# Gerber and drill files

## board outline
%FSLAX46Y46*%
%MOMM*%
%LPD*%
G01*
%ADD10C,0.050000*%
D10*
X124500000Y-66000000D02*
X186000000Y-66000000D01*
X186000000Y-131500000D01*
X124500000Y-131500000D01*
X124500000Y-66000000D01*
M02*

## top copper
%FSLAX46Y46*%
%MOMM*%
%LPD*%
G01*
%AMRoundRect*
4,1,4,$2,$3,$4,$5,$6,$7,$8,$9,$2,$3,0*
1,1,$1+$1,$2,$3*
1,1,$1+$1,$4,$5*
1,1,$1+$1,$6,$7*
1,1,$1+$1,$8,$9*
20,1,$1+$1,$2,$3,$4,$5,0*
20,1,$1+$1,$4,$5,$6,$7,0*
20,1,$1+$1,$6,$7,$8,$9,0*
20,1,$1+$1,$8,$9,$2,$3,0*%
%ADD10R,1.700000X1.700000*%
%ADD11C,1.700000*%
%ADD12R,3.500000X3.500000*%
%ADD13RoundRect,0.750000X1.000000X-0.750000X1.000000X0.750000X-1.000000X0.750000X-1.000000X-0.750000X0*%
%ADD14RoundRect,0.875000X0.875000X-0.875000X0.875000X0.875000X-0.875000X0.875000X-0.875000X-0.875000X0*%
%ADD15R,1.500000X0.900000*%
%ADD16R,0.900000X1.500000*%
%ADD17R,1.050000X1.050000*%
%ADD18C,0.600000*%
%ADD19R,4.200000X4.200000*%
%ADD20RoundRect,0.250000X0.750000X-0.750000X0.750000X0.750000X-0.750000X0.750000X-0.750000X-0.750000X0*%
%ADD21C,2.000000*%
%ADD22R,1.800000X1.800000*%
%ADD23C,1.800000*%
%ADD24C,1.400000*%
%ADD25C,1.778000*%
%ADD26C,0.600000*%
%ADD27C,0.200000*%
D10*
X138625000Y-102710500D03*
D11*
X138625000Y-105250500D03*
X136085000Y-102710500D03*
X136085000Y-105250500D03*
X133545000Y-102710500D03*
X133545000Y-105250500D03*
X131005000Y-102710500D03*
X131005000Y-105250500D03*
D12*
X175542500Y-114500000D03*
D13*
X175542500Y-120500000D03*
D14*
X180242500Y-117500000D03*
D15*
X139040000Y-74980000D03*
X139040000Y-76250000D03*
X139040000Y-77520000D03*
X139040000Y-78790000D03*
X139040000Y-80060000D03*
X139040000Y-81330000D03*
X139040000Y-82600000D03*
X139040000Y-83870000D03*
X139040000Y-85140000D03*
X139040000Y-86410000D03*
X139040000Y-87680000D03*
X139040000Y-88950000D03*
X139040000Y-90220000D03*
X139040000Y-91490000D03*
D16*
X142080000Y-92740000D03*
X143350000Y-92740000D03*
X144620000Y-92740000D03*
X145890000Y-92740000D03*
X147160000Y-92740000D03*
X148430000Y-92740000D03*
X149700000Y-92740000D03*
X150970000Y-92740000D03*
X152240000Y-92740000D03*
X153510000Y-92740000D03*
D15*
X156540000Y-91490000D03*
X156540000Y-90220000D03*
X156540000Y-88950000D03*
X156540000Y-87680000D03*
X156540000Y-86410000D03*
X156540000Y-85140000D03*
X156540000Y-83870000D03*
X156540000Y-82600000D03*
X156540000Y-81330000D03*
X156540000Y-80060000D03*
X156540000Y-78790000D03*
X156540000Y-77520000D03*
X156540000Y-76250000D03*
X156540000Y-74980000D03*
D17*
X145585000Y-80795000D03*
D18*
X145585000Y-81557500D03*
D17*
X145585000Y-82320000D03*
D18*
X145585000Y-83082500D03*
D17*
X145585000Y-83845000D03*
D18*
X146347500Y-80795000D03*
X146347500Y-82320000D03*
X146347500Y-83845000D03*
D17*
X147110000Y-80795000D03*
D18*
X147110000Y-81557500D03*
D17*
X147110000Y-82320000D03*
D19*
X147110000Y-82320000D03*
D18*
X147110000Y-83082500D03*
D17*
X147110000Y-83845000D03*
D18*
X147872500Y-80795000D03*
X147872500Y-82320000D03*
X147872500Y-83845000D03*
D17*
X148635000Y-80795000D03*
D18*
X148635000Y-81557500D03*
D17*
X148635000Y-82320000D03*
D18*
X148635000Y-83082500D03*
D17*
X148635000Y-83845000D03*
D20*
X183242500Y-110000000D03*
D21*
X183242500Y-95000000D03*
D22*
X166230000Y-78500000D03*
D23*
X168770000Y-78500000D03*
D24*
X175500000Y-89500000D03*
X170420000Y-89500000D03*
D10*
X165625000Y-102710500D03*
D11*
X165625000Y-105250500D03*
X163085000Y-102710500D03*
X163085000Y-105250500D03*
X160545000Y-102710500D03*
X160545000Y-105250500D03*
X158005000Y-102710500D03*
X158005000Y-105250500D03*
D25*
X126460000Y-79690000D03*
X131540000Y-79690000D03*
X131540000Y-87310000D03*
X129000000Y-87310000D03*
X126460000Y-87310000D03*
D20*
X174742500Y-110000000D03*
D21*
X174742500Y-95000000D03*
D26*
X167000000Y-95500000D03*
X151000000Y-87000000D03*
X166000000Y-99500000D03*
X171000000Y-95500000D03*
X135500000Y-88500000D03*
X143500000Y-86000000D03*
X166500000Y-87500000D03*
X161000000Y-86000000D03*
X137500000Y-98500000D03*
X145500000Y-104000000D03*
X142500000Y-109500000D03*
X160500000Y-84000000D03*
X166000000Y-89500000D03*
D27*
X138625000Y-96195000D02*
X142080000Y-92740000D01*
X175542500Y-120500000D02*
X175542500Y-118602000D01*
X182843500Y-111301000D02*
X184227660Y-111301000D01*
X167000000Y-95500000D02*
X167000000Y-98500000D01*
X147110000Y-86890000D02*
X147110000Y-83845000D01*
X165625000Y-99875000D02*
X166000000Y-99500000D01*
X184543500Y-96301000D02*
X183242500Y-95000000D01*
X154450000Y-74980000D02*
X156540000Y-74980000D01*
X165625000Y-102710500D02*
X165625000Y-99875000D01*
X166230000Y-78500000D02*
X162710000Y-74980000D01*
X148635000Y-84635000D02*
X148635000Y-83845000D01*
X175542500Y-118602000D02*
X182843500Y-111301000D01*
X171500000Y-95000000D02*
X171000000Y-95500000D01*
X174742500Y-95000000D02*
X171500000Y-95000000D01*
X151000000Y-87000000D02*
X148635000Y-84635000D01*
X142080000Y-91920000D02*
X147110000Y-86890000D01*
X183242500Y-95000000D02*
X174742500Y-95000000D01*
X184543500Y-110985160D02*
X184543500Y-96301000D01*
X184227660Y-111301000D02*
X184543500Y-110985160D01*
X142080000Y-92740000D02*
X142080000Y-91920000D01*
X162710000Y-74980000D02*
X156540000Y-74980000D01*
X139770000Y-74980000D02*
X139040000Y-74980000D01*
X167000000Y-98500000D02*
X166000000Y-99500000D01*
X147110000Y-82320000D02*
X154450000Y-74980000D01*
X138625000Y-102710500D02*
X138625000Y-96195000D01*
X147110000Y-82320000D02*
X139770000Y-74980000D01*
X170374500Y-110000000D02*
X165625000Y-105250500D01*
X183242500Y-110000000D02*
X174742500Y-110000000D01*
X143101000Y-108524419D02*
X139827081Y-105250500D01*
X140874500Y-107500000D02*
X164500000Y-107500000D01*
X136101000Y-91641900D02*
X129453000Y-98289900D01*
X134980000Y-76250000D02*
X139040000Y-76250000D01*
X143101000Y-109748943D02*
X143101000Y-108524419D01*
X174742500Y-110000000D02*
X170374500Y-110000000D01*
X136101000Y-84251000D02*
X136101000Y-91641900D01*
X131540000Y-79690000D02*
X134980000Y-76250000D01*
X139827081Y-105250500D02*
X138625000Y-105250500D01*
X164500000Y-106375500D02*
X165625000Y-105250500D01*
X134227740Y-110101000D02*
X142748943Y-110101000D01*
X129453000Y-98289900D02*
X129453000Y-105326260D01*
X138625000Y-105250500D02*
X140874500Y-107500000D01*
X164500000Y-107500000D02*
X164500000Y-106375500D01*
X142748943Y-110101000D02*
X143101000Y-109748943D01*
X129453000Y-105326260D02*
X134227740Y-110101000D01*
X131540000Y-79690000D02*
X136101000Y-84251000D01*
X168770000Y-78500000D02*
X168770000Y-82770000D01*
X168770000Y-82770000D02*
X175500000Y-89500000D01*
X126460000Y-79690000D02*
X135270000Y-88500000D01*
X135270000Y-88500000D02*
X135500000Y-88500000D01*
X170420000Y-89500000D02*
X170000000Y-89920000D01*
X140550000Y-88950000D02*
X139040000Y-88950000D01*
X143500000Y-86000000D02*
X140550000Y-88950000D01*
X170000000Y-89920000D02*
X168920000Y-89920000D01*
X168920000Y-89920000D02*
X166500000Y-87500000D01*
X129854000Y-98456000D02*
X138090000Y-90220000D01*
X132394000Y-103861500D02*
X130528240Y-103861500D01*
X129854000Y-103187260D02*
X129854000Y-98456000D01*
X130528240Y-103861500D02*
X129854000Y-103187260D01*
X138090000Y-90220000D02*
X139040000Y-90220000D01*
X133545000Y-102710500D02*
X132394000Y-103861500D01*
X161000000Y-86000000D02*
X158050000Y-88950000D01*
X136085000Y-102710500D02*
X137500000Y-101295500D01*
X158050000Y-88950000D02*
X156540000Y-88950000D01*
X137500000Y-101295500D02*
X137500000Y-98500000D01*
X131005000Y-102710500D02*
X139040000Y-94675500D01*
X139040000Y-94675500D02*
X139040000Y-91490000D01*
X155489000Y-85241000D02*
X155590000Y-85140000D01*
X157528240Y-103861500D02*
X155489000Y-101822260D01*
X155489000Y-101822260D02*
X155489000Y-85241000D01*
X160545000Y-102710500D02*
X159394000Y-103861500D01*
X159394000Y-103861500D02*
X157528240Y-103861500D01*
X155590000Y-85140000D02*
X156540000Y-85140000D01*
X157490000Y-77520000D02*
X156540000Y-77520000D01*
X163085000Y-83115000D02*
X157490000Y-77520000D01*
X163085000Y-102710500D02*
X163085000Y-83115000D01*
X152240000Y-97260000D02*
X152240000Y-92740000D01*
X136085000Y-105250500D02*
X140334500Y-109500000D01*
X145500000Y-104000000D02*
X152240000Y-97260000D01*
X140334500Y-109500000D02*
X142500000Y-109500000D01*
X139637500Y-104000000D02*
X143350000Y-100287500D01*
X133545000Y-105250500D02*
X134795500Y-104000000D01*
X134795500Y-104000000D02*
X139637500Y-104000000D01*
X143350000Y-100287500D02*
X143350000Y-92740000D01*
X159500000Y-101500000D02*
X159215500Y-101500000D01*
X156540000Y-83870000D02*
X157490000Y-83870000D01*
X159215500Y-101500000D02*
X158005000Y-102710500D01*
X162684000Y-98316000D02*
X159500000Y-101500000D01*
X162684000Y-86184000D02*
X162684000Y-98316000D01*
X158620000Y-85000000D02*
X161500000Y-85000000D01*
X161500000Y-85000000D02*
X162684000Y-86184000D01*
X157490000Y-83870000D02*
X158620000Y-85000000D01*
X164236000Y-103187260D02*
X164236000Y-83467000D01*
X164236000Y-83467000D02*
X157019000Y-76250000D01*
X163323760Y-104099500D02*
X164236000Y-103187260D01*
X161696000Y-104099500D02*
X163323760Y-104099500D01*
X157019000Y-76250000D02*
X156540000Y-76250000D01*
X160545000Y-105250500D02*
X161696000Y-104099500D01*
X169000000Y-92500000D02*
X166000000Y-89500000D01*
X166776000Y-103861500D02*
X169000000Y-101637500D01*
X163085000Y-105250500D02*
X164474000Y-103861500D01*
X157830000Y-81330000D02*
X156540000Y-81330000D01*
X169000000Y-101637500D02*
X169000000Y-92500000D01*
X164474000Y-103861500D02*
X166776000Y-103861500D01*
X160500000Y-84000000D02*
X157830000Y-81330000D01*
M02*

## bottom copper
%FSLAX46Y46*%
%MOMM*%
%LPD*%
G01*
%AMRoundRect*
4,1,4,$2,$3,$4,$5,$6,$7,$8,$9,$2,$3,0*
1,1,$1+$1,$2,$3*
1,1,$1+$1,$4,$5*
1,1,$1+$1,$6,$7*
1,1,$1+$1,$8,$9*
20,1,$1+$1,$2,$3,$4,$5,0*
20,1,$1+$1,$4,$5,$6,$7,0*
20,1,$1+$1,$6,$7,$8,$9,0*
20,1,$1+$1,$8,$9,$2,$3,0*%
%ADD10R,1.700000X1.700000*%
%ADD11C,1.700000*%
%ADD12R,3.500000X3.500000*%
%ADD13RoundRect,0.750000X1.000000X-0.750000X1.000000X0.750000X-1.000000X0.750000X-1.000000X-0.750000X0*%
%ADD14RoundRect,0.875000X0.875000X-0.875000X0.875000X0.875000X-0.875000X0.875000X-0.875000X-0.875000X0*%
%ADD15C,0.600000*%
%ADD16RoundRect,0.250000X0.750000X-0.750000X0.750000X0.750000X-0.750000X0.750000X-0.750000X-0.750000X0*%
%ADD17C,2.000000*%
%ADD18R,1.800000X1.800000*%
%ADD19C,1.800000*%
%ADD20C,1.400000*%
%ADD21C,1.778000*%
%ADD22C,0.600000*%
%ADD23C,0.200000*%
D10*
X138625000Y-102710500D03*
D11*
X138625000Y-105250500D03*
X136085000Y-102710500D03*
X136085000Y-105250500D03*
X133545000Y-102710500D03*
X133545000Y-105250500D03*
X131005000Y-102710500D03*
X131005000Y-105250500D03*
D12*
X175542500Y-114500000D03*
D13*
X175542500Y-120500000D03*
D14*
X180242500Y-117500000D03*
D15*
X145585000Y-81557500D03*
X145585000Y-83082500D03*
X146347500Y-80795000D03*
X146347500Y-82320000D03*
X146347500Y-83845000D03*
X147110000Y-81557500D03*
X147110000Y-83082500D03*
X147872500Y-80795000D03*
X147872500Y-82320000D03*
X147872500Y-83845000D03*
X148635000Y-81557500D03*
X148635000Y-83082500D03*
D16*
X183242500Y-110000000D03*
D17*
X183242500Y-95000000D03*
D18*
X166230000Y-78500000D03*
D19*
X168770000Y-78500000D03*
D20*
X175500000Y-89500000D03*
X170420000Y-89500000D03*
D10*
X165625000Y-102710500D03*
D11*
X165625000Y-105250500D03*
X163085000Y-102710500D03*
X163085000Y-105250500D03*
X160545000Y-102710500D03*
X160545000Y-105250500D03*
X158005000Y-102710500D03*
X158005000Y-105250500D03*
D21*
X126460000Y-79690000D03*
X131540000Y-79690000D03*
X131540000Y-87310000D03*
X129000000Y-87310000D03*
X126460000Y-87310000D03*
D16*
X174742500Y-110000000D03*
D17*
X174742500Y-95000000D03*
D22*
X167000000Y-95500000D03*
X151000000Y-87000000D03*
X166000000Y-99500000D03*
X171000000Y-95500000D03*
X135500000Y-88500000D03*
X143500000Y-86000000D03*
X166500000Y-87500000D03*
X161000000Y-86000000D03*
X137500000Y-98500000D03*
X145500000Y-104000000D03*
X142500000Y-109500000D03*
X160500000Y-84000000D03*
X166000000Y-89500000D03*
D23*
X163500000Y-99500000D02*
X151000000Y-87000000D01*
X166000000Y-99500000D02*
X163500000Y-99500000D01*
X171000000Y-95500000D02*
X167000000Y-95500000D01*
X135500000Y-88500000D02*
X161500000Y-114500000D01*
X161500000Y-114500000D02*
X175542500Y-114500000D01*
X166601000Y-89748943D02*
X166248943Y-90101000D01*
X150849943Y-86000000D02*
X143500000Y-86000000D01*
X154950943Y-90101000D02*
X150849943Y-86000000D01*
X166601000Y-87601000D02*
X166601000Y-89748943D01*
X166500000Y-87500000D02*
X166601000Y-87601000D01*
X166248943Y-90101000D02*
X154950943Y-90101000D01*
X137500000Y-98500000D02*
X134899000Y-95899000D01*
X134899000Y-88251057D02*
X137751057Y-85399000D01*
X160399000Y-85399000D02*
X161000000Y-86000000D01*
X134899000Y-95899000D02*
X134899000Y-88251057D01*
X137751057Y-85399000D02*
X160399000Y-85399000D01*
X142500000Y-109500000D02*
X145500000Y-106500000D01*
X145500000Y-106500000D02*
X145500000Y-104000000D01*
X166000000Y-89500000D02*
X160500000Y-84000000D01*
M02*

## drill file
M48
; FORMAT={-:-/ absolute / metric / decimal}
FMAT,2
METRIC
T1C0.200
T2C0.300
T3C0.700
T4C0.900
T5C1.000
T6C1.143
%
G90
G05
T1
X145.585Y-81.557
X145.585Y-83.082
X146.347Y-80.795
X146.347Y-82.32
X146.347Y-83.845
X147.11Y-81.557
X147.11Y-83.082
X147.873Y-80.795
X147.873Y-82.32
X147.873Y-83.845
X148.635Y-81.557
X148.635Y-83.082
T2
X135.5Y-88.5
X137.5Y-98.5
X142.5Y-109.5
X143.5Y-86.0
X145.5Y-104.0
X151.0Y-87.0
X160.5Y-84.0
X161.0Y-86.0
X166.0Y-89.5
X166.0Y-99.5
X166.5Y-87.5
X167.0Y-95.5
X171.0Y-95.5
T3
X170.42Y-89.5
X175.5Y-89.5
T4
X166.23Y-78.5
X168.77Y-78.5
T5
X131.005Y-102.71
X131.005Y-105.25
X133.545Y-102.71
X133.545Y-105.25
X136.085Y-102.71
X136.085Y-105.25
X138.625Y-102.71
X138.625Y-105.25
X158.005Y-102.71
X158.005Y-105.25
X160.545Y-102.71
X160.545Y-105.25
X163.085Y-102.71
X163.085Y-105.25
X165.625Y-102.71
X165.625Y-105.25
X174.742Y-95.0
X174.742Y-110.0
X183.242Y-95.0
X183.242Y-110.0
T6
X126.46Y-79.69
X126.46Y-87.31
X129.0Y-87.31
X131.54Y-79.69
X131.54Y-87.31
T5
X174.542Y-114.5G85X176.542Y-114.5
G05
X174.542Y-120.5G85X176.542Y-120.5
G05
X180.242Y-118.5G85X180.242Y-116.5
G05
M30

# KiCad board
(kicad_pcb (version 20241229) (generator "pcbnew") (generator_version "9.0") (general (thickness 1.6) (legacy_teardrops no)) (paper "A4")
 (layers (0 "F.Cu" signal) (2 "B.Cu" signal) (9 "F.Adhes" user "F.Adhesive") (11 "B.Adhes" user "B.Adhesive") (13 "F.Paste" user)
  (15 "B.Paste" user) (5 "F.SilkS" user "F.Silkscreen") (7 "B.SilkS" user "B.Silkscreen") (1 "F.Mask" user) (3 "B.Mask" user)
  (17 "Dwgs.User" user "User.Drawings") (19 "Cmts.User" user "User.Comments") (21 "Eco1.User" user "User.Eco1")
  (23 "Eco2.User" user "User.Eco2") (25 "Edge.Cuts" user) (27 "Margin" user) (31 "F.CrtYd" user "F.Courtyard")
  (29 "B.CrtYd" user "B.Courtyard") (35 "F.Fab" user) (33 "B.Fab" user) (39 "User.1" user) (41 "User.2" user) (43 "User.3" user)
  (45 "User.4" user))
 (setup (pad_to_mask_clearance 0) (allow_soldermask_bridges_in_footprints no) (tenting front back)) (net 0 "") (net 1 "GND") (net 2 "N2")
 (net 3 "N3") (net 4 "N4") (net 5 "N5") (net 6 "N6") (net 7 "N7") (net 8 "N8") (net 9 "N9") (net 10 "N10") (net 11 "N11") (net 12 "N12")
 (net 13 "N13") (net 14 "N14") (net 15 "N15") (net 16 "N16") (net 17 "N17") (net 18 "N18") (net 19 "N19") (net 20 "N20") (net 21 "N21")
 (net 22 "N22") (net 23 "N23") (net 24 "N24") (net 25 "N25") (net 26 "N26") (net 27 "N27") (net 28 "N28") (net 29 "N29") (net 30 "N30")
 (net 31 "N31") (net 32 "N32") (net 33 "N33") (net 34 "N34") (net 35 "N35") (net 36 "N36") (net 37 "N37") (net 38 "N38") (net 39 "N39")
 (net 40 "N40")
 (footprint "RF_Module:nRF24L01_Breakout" (layer "F.Cu") (at 138.625 102.7105 -90)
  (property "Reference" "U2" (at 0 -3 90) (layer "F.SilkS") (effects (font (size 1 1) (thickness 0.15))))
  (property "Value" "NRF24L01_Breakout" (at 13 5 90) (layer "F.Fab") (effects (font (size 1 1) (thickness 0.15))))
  (pad "1" thru_hole rect (at 0 0 270) (size 1.7 1.7) (drill 1) (layers "*.Cu" "*.Mask") (remove_unused_layers no) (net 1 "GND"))
  (pad "2" thru_hole circle (at 2.54 0 270) (size 1.7 1.7) (drill 1) (layers "*.Cu" "*.Mask") (remove_unused_layers no) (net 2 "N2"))
  (pad "3" thru_hole circle (at 0 2.54 270) (size 1.7 1.7) (drill 1) (layers "*.Cu" "*.Mask") (remove_unused_layers no) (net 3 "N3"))
  (pad "4" thru_hole circle (at 2.54 2.54 270) (size 1.7 1.7) (drill 1) (layers "*.Cu" "*.Mask") (remove_unused_layers no) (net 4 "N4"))
  (pad "5" thru_hole circle (at 0 5.08 270) (size 1.7 1.7) (drill 1) (layers "*.Cu" "*.Mask") (remove_unused_layers no) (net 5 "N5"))
  (pad "6" thru_hole circle (at 2.54 5.08 270) (size 1.7 1.7) (drill 1) (layers "*.Cu" "*.Mask") (remove_unused_layers no) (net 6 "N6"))
  (pad "7" thru_hole circle (at 0 7.62 270) (size 1.7 1.7) (drill 1) (layers "*.Cu" "*.Mask") (remove_unused_layers no) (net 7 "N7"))
  (pad "8" thru_hole circle (at 2.54 7.62 270) (size 1.7 1.7) (drill 1) (layers "*.Cu" "*.Mask") (remove_unused_layers no) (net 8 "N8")))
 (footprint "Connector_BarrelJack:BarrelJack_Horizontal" (layer "F.Cu") (at 175.5425 114.5 90)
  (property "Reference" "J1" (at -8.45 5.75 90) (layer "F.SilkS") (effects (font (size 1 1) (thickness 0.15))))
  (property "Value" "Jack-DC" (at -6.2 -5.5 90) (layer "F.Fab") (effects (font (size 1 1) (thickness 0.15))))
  (pad "1" thru_hole rect (at 0 0 90) (size 3.5 3.5) (drill oval 1 3) (layers "*.Cu" "*.Mask") (remove_unused_layers no) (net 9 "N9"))
  (pad "2" thru_hole roundrect (at -6 0 90) (size 3 3.5) (drill oval 1 3) (layers "*.Cu" "*.Mask") (remove_unused_layers no)
   (roundrect_rratio 0.25) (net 1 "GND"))
  (pad "3" thru_hole roundrect (at -3 4.7 90) (size 3.5 3.5) (drill oval 3 1) (layers "*.Cu" "*.Mask") (remove_unused_layers no)
   (roundrect_rratio 0.25)))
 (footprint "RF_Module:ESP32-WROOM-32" (layer "F.Cu") (at 147.79 83.23)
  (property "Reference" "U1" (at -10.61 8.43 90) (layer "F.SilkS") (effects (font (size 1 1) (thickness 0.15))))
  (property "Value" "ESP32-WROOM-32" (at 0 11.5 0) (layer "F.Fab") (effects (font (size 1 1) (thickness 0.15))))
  (pad "1" smd rect (at -8.75 -8.25) (size 1.5 0.9) (layers "F.Cu" "F.Mask" "F.Paste") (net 1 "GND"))
  (pad "2" smd rect (at -8.75 -6.98) (size 1.5 0.9) (layers "F.Cu" "F.Mask" "F.Paste") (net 2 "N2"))
  (pad "3" smd rect (at -8.75 -5.71) (size 1.5 0.9) (layers "F.Cu" "F.Mask" "F.Paste") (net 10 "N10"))
  (pad "4" smd rect (at -8.75 -4.44) (size 1.5 0.9) (layers "F.Cu" "F.Mask" "F.Paste") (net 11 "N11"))
  (pad "5" smd rect (at -8.75 -3.17) (size 1.5 0.9) (layers "F.Cu" "F.Mask" "F.Paste") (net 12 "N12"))
  (pad "6" smd rect (at -8.75 -1.9) (size 1.5 0.9) (layers "F.Cu" "F.Mask" "F.Paste") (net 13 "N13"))
  (pad "7" smd rect (at -8.75 -0.63) (size 1.5 0.9) (layers "F.Cu" "F.Mask" "F.Paste") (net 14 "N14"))
  (pad "8" smd rect (at -8.75 0.64) (size 1.5 0.9) (layers "F.Cu" "F.Mask" "F.Paste") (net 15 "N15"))
  (pad "9" smd rect (at -8.75 1.91) (size 1.5 0.9) (layers "F.Cu" "F.Mask" "F.Paste") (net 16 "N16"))
  (pad "10" smd rect (at -8.75 3.18) (size 1.5 0.9) (layers "F.Cu" "F.Mask" "F.Paste") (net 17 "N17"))
  (pad "11" smd rect (at -8.75 4.45) (size 1.5 0.9) (layers "F.Cu" "F.Mask" "F.Paste") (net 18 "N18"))
  (pad "12" smd rect (at -8.75 5.72) (size 1.5 0.9) (layers "F.Cu" "F.Mask" "F.Paste") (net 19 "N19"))
  (pad "13" smd rect (at -8.75 6.99) (size 1.5 0.9) (layers "F.Cu" "F.Mask" "F.Paste") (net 5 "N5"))
  (pad "14" smd rect (at -8.75 8.26) (size 1.5 0.9) (layers "F.Cu" "F.Mask" "F.Paste") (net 7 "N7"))
  (pad "15" smd rect (at -5.71 9.51 90) (size 1.5 0.9) (layers "F.Cu" "F.Mask" "F.Paste") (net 1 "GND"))
  (pad "16" smd rect (at -4.44 9.51 90) (size 1.5 0.9) (layers "F.Cu" "F.Mask" "F.Paste") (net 6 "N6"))
  (pad "17" smd rect (at -3.17 9.51 90) (size 1.5 0.9) (layers "F.Cu" "F.Mask" "F.Paste") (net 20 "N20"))
  (pad "18" smd rect (at -1.9 9.51 90) (size 1.5 0.9) (layers "F.Cu" "F.Mask" "F.Paste") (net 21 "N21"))
  (pad "19" smd rect (at -0.63 9.51 90) (size 1.5 0.9) (layers "F.Cu" "F.Mask" "F.Paste") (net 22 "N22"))
  (pad "20" smd rect (at 0.64 9.51 90) (size 1.5 0.9) (layers "F.Cu" "F.Mask" "F.Paste") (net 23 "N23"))
  (pad "21" smd rect (at 1.91 9.51 90) (size 1.5 0.9) (layers "F.Cu" "F.Mask" "F.Paste") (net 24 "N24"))
  (pad "22" smd rect (at 3.18 9.51 90) (size 1.5 0.9) (layers "F.Cu" "F.Mask" "F.Paste") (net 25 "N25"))
  (pad "23" smd rect (at 4.45 9.51 90) (size 1.5 0.9) (layers "F.Cu" "F.Mask" "F.Paste") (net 4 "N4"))
  (pad "24" smd rect (at 5.72 9.51 90) (size 1.5 0.9) (layers "F.Cu" "F.Mask" "F.Paste") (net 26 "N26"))
  (pad "25" smd rect (at 8.75 8.26) (size 1.5 0.9) (layers "F.Cu" "F.Mask" "F.Paste") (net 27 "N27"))
  (pad "26" smd rect (at 8.75 6.99) (size 1.5 0.9) (layers "F.Cu" "F.Mask" "F.Paste") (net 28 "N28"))
  (pad "27" smd rect (at 8.75 5.72) (size 1.5 0.9) (layers "F.Cu" "F.Mask" "F.Paste") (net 3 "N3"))
  (pad "28" smd rect (at 8.75 4.45) (size 1.5 0.9) (layers "F.Cu" "F.Mask" "F.Paste") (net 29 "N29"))
  (pad "29" smd rect (at 8.75 3.18) (size 1.5 0.9) (layers "F.Cu" "F.Mask" "F.Paste") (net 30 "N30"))
  (pad "30" smd rect (at 8.75 1.91) (size 1.5 0.9) (layers "F.Cu" "F.Mask" "F.Paste") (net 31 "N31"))
  (pad "31" smd rect (at 8.75 0.64) (size 1.5 0.9) (layers "F.Cu" "F.Mask" "F.Paste") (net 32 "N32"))
  (pad "32" smd rect (at 8.75 -0.63) (size 1.5 0.9) (layers "F.Cu" "F.Mask" "F.Paste") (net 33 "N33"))
  (pad "33" smd rect (at 8.75 -1.9) (size 1.5 0.9) (layers "F.Cu" "F.Mask" "F.Paste") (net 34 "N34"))
  (pad "34" smd rect (at 8.75 -3.17) (size 1.5 0.9) (layers "F.Cu" "F.Mask" "F.Paste") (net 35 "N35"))
  (pad "35" smd rect (at 8.75 -4.44) (size 1.5 0.9) (layers "F.Cu" "F.Mask" "F.Paste") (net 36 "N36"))
  (pad "36" smd rect (at 8.75 -5.71) (size 1.5 0.9) (layers "F.Cu" "F.Mask" "F.Paste") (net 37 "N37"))
  (pad "37" smd rect (at 8.75 -6.98) (size 1.5 0.9) (layers "F.Cu" "F.Mask" "F.Paste") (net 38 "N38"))
  (pad "38" smd rect (at 8.75 -8.25) (size 1.5 0.9) (layers "F.Cu" "F.Mask" "F.Paste") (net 1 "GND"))
  (pad "39" smd rect (at -2.205 -2.435) (size 1.05 1.05) (layers "F.Cu" "F.Paste") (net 1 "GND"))
  (pad "39" thru_hole circle (at -2.205 -1.6725) (size 0.6 0.6) (drill 0.2) (layers "*.Cu" "F.Mask") (remove_unused_layers no) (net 1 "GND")
   (zone_connect 2))
  (pad "39" smd rect (at -2.205 -0.91) (size 1.05 1.05) (layers "F.Cu" "F.Paste") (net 1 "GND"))
  (pad "39" thru_hole circle (at -2.205 -0.1475) (size 0.6 0.6) (drill 0.2) (layers "*.Cu" "F.Mask") (remove_unused_layers no) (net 1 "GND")
   (zone_connect 2))
  (pad "39" smd rect (at -2.205 0.615) (size 1.05 1.05) (layers "F.Cu" "F.Paste") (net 1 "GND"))
  (pad "39" thru_hole circle (at -1.4425 -2.435) (size 0.6 0.6) (drill 0.2) (layers "*.Cu" "F.Mask") (remove_unused_layers no) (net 1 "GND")
   (zone_connect 2))
  (pad "39" thru_hole circle (at -1.4425 -0.91) (size 0.6 0.6) (drill 0.2) (layers "*.Cu" "F.Mask") (remove_unused_layers no) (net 1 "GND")
   (zone_connect 2))
  (pad "39" thru_hole circle (at -1.4425 0.615) (size 0.6 0.6) (drill 0.2) (layers "*.Cu" "F.Mask") (remove_unused_layers no) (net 1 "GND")
   (zone_connect 2))
  (pad "39" smd rect (at -0.68 -2.435) (size 1.05 1.05) (layers "F.Cu" "F.Paste") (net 1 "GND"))
  (pad "39" thru_hole circle (at -0.68 -1.6725) (size 0.6 0.6) (drill 0.2) (layers "*.Cu" "F.Mask") (remove_unused_layers no) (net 1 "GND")
   (zone_connect 2))
  (pad "39" smd rect (at -0.68 -0.91) (size 1.05 1.05) (layers "F.Cu" "F.Paste") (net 1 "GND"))
  (pad "39" smd rect (at -0.68 -0.91) (size 4.2 4.2) (layers "F.Cu" "F.Mask") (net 1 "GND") (zone_connect 2))
  (pad "39" thru_hole circle (at -0.68 -0.1475) (size 0.6 0.6) (drill 0.2) (layers "*.Cu" "F.Mask") (remove_unused_layers no) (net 1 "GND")
   (zone_connect 2))
  (pad "39" smd rect (at -0.68 0.615) (size 1.05 1.05) (layers "F.Cu" "F.Paste") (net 1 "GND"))
  (pad "39" thru_hole circle (at 0.0825 -2.435) (size 0.6 0.6) (drill 0.2) (layers "*.Cu" "F.Mask") (remove_unused_layers no) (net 1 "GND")
   (zone_connect 2))
  (pad "39" thru_hole circle (at 0.0825 -0.91) (size 0.6 0.6) (drill 0.2) (layers "*.Cu" "F.Mask") (remove_unused_layers no) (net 1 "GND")
   (zone_connect 2))
  (pad "39" thru_hole circle (at 0.0825 0.615) (size 0.6 0.6) (drill 0.2) (layers "*.Cu" "F.Mask") (remove_unused_layers no) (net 1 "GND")
   (zone_connect 2))
  (pad "39" smd rect (at 0.845 -2.435) (size 1.05 1.05) (layers "F.Cu" "F.Paste") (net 1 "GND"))
  (pad "39" thru_hole circle (at 0.845 -1.6725) (size 0.6 0.6) (drill 0.2) (layers "*.Cu" "F.Mask") (remove_unused_layers no) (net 1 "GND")
   (zone_connect 2))
  (pad "39" smd rect (at 0.845 -0.91) (size 1.05 1.05) (layers "F.Cu" "F.Paste") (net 1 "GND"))
  (pad "39" thru_hole circle (at 0.845 -0.1475) (size 0.6 0.6) (drill 0.2) (layers "*.Cu" "F.Mask") (remove_unused_layers no) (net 1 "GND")
   (zone_connect 2))
  (pad "39" smd rect (at 0.845 0.615) (size 1.05 1.05) (layers "F.Cu" "F.Paste") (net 1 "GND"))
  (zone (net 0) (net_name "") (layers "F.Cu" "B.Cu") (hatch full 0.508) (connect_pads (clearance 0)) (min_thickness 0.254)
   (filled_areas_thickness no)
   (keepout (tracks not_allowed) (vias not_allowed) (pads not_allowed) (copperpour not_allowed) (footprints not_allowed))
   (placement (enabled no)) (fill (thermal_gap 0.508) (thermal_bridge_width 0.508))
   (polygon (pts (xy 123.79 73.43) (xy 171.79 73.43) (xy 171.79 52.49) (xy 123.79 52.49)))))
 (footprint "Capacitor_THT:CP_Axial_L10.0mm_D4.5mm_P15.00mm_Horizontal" (layer "F.Cu") (at 183.2425 110 90)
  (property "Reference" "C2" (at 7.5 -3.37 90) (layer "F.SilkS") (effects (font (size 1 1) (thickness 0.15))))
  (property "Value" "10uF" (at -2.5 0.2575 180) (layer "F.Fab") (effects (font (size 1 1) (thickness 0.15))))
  (pad "1" thru_hole roundrect (at 0 0 90) (size 2 2) (drill 1) (layers "*.Cu" "*.Mask") (remove_unused_layers no) (roundrect_rratio 0.125)
   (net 2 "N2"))
  (pad "2" thru_hole circle (at 15 0 90) (size 2 2) (drill 1) (layers "*.Cu" "*.Mask") (remove_unused_layers no) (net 1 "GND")))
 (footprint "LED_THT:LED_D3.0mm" (layer "F.Cu") (at 166.23 78.5)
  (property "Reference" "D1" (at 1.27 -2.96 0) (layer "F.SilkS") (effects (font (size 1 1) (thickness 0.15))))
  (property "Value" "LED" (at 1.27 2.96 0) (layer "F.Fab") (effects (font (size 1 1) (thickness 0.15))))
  (pad "1" thru_hole rect (at 0 0) (size 1.8 1.8) (drill 0.9) (layers "*.Cu" "*.Mask") (remove_unused_layers no) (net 1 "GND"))
  (pad "2" thru_hole circle (at 2.54 0) (size 1.8 1.8) (drill 0.9) (layers "*.Cu" "*.Mask") (remove_unused_layers no) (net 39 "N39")))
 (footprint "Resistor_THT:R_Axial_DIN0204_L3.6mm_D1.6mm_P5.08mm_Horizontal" (layer "F.Cu") (at 175.5 89.5 180)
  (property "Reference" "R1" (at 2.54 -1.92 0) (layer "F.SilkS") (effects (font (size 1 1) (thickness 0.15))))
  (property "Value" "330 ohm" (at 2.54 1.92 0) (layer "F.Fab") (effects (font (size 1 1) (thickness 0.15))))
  (pad "1" thru_hole circle (at 0 0 180) (size 1.4 1.4) (drill 0.7) (layers "*.Cu" "*.Mask") (remove_unused_layers no) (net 39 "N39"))
  (pad "2" thru_hole circle (at 5.08 0 180) (size 1.4 1.4) (drill 0.7) (layers "*.Cu" "*.Mask") (remove_unused_layers no) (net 19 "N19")))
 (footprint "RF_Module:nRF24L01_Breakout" (layer "F.Cu") (at 165.625 102.7105 -90)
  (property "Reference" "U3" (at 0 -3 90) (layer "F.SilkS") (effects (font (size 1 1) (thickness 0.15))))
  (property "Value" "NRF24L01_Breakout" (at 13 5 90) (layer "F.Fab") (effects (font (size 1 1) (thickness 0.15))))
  (pad "1" thru_hole rect (at 0 0 270) (size 1.7 1.7) (drill 1) (layers "*.Cu" "*.Mask") (remove_unused_layers no) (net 1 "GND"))
  (pad "2" thru_hole circle (at 2.54 0 270) (size 1.7 1.7) (drill 1) (layers "*.Cu" "*.Mask") (remove_unused_layers no) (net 2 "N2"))
  (pad "3" thru_hole circle (at 0 2.54 270) (size 1.7 1.7) (drill 1) (layers "*.Cu" "*.Mask") (remove_unused_layers no) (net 37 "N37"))
  (pad "4" thru_hole circle (at 2.54 2.54 270) (size 1.7 1.7) (drill 1) (layers "*.Cu" "*.Mask") (remove_unused_layers no) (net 34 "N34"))
  (pad "5" thru_hole circle (at 0 5.08 270) (size 1.7 1.7) (drill 1) (layers "*.Cu" "*.Mask") (remove_unused_layers no) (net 31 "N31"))
  (pad "6" thru_hole circle (at 2.54 5.08 270) (size 1.7 1.7) (drill 1) (layers "*.Cu" "*.Mask") (remove_unused_layers no) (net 38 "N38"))
  (pad "7" thru_hole circle (at 0 7.62 270) (size 1.7 1.7) (drill 1) (layers "*.Cu" "*.Mask") (remove_unused_layers no) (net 32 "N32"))
  (pad "8" thru_hole circle (at 2.54 7.62 270) (size 1.7 1.7) (drill 1) (layers "*.Cu" "*.Mask") (remove_unused_layers no) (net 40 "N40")))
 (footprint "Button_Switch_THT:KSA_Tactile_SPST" (layer "F.Cu") (at 126.46 79.69)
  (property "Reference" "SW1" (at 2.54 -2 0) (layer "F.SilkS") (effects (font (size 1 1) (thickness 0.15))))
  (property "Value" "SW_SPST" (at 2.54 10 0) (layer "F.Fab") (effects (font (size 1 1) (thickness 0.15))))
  (pad "1" thru_hole circle (at 0 0) (size 1.778 1.778) (drill 1.143) (layers "*.Cu" "*.Mask") (remove_unused_layers no) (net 9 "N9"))
  (pad "2" thru_hole circle (at 5.08 0) (size 1.778 1.778) (drill 1.143) (layers "*.Cu" "*.Mask") (remove_unused_layers no) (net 2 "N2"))
  (pad "3" thru_hole circle (at 5.08 7.62) (size 1.778 1.778) (drill 1.143) (layers "*.Cu" "*.Mask") (remove_unused_layers no))
  (pad "4" thru_hole circle (at 2.54 7.62) (size 1.778 1.778) (drill 1.143) (layers "*.Cu" "*.Mask") (remove_unused_layers no))
  (pad "5" thru_hole circle (at 0 7.62) (size 1.778 1.778) (drill 1.143) (layers "*.Cu" "*.Mask") (remove_unused_layers no)))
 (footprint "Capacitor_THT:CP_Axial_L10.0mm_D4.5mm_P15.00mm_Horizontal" (layer "F.Cu") (at 174.7425 110 90)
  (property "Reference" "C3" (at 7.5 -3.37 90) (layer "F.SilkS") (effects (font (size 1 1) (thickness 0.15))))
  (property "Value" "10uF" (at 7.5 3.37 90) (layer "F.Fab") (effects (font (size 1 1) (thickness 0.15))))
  (pad "1" thru_hole roundrect (at 0 0 90) (size 2 2) (drill 1) (layers "*.Cu" "*.Mask") (remove_unused_layers no) (roundrect_rratio 0.125)
   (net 2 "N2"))
  (pad "2" thru_hole circle (at 15 0 90) (size 2 2) (drill 1) (layers "*.Cu" "*.Mask") (remove_unused_layers no) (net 1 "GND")))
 (gr_rect (start 124.5 66) (end 186 131.5) (stroke (width 0.05) (type default)) (fill no) (layer "Edge.Cuts"))
 (segment (start 138.625 96.195) (end 142.08 92.74) (width 0.2) (layer "F.Cu") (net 1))
 (segment (start 175.5425 120.5) (end 175.5425 118.602) (width 0.2) (layer "F.Cu") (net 1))
 (segment (start 182.8435 111.301) (end 184.22766 111.301) (width 0.2) (layer "F.Cu") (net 1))
 (segment (start 167 95.5) (end 167 98.5) (width 0.2) (layer "F.Cu") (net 1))
 (segment (start 147.11 86.89) (end 147.11 83.845) (width 0.2) (layer "F.Cu") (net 1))
 (segment (start 165.625 99.875) (end 166 99.5) (width 0.2) (layer "F.Cu") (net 1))
 (segment (start 184.5435 96.301) (end 183.2425 95) (width 0.2) (layer "F.Cu") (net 1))
 (segment (start 154.45 74.98) (end 156.54 74.98) (width 0.2) (layer "F.Cu") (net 1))
 (segment (start 165.625 102.7105) (end 165.625 99.875) (width 0.2) (layer "F.Cu") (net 1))
 (segment (start 166.23 78.5) (end 162.71 74.98) (width 0.2) (layer "F.Cu") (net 1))
 (segment (start 148.635 84.635) (end 148.635 83.845) (width 0.2) (layer "F.Cu") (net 1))
 (segment (start 175.5425 118.602) (end 182.8435 111.301) (width 0.2) (layer "F.Cu") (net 1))
 (segment (start 171.5 95) (end 171 95.5) (width 0.2) (layer "F.Cu") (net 1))
 (segment (start 174.7425 95) (end 171.5 95) (width 0.2) (layer "F.Cu") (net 1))
 (segment (start 151 87) (end 148.635 84.635) (width 0.2) (layer "F.Cu") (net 1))
 (segment (start 142.08 91.92) (end 147.11 86.89) (width 0.2) (layer "F.Cu") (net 1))
 (segment (start 183.2425 95) (end 174.7425 95) (width 0.2) (layer "F.Cu") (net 1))
 (segment (start 184.5435 110.98516) (end 184.5435 96.301) (width 0.2) (layer "F.Cu") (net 1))
 (segment (start 184.22766 111.301) (end 184.5435 110.98516) (width 0.2) (layer "F.Cu") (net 1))
 (segment (start 142.08 92.74) (end 142.08 91.92) (width 0.2) (layer "F.Cu") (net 1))
 (segment (start 162.71 74.98) (end 156.54 74.98) (width 0.2) (layer "F.Cu") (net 1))
 (segment (start 139.77 74.98) (end 139.04 74.98) (width 0.2) (layer "F.Cu") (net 1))
 (segment (start 167 98.5) (end 166 99.5) (width 0.2) (layer "F.Cu") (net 1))
 (segment (start 147.11 82.32) (end 154.45 74.98) (width 0.2) (layer "F.Cu") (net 1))
 (segment (start 138.625 102.7105) (end 138.625 96.195) (width 0.2) (layer "F.Cu") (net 1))
 (segment (start 147.11 82.32) (end 139.77 74.98) (width 0.2) (layer "F.Cu") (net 1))
 (via (at 167 95.5) (size 0.6) (drill 0.3) (layers "F.Cu" "B.Cu") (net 1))
 (via (at 151 87) (size 0.6) (drill 0.3) (layers "F.Cu" "B.Cu") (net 1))
 (via (at 166 99.5) (size 0.6) (drill 0.3) (layers "F.Cu" "B.Cu") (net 1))
 (via (at 171 95.5) (size 0.6) (drill 0.3) (layers "F.Cu" "B.Cu") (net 1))
 (segment (start 163.5 99.5) (end 151 87) (width 0.2) (layer "B.Cu") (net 1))
 (segment (start 166 99.5) (end 163.5 99.5) (width 0.2) (layer "B.Cu") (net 1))
 (segment (start 171 95.5) (end 167 95.5) (width 0.2) (layer "B.Cu") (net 1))
 (segment (start 170.3745 110) (end 165.625 105.2505) (width 0.2) (layer "F.Cu") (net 2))
 (segment (start 183.2425 110) (end 174.7425 110) (width 0.2) (layer "F.Cu") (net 2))
 (segment (start 143.101 108.524419) (end 139.827081 105.2505) (width 0.2) (layer "F.Cu") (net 2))
 (segment (start 140.8745 107.5) (end 164.5 107.5) (width 0.2) (layer "F.Cu") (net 2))
 (segment (start 136.101 91.6419) (end 129.453 98.2899) (width 0.2) (layer "F.Cu") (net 2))
 (segment (start 134.98 76.25) (end 139.04 76.25) (width 0.2) (layer "F.Cu") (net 2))
 (segment (start 143.101 109.748943) (end 143.101 108.524419) (width 0.2) (layer "F.Cu") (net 2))
 (segment (start 174.7425 110) (end 170.3745 110) (width 0.2) (layer "F.Cu") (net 2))
 (segment (start 136.101 84.251) (end 136.101 91.6419) (width 0.2) (layer "F.Cu") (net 2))
 (segment (start 131.54 79.69) (end 134.98 76.25) (width 0.2) (layer "F.Cu") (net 2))
 (segment (start 139.827081 105.2505) (end 138.625 105.2505) (width 0.2) (layer "F.Cu") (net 2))
 (segment (start 164.5 106.3755) (end 165.625 105.2505) (width 0.2) (layer "F.Cu") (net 2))
 (segment (start 134.22774 110.101) (end 142.748943 110.101) (width 0.2) (layer "F.Cu") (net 2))
 (segment (start 129.453 98.2899) (end 129.453 105.32626) (width 0.2) (layer "F.Cu") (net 2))
 (segment (start 138.625 105.2505) (end 140.8745 107.5) (width 0.2) (layer "F.Cu") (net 2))
 (segment (start 164.5 107.5) (end 164.5 106.3755) (width 0.2) (layer "F.Cu") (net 2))
 (segment (start 142.748943 110.101) (end 143.101 109.748943) (width 0.2) (layer "F.Cu") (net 2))
 (segment (start 129.453 105.32626) (end 134.22774 110.101) (width 0.2) (layer "F.Cu") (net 2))
 (segment (start 131.54 79.69) (end 136.101 84.251) (width 0.2) (layer "F.Cu") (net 2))
 (segment (start 168.77 78.5) (end 168.77 82.77) (width 0.2) (layer "F.Cu") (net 39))
 (segment (start 168.77 82.77) (end 175.5 89.5) (width 0.2) (layer "F.Cu") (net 39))
 (segment (start 126.46 79.69) (end 135.27 88.5) (width 0.2) (layer "F.Cu") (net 9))
 (segment (start 135.27 88.5) (end 135.5 88.5) (width 0.2) (layer "F.Cu") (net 9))
 (via (at 135.5 88.5) (size 0.6) (drill 0.3) (layers "F.Cu" "B.Cu") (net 9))
 (segment (start 135.5 88.5) (end 161.5 114.5) (width 0.2) (layer "B.Cu") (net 9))
 (segment (start 161.5 114.5) (end 175.5425 114.5) (width 0.2) (layer "B.Cu") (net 9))
 (segment (start 170.42 89.5) (end 170 89.92) (width 0.2) (layer "F.Cu") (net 19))
 (segment (start 140.55 88.95) (end 139.04 88.95) (width 0.2) (layer "F.Cu") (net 19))
 (segment (start 143.5 86) (end 140.55 88.95) (width 0.2) (layer "F.Cu") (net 19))
 (segment (start 170 89.92) (end 168.92 89.92) (width 0.2) (layer "F.Cu") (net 19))
 (segment (start 168.92 89.92) (end 166.5 87.5) (width 0.2) (layer "F.Cu") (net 19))
 (via (at 143.5 86) (size 0.6) (drill 0.3) (layers "F.Cu" "B.Cu") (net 19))
 (via (at 166.5 87.5) (size 0.6) (drill 0.3) (layers "F.Cu" "B.Cu") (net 19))
 (segment (start 166.601 89.748943) (end 166.248943 90.101) (width 0.2) (layer "B.Cu") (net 19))
 (segment (start 150.849943 86) (end 143.5 86) (width 0.2) (layer "B.Cu") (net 19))
 (segment (start 154.950943 90.101) (end 150.849943 86) (width 0.2) (layer "B.Cu") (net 19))
 (segment (start 166.601 87.601) (end 166.601 89.748943) (width 0.2) (layer "B.Cu") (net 19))
 (segment (start 166.5 87.5) (end 166.601 87.601) (width 0.2) (layer "B.Cu") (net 19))
 (segment (start 166.248943 90.101) (end 154.950943 90.101) (width 0.2) (layer "B.Cu") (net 19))
 (segment (start 129.854 98.456) (end 138.09 90.22) (width 0.2) (layer "F.Cu") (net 5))
 (segment (start 132.394 103.8615) (end 130.52824 103.8615) (width 0.2) (layer "F.Cu") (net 5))
 (segment (start 129.854 103.18726) (end 129.854 98.456) (width 0.2) (layer "F.Cu") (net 5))
 (segment (start 130.52824 103.8615) (end 129.854 103.18726) (width 0.2) (layer "F.Cu") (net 5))
 (segment (start 138.09 90.22) (end 139.04 90.22) (width 0.2) (layer "F.Cu") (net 5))
 (segment (start 133.545 102.7105) (end 132.394 103.8615) (width 0.2) (layer "F.Cu") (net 5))
 (segment (start 161 86) (end 158.05 88.95) (width 0.2) (layer "F.Cu") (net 3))
 (segment (start 136.085 102.7105) (end 137.5 101.2955) (width 0.2) (layer "F.Cu") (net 3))
 (segment (start 158.05 88.95) (end 156.54 88.95) (width 0.2) (layer "F.Cu") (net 3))
 (segment (start 137.5 101.2955) (end 137.5 98.5) (width 0.2) (layer "F.Cu") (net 3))
 (via (at 161 86) (size 0.6) (drill 0.3) (layers "F.Cu" "B.Cu") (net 3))
 (via (at 137.5 98.5) (size 0.6) (drill 0.3) (layers "F.Cu" "B.Cu") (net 3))
 (segment (start 137.5 98.5) (end 134.899 95.899) (width 0.2) (layer "B.Cu") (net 3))
 (segment (start 134.899 88.251057) (end 137.751057 85.399) (width 0.2) (layer "B.Cu") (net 3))
 (segment (start 160.399 85.399) (end 161 86) (width 0.2) (layer "B.Cu") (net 3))
 (segment (start 134.899 95.899) (end 134.899 88.251057) (width 0.2) (layer "B.Cu") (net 3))
 (segment (start 137.751057 85.399) (end 160.399 85.399) (width 0.2) (layer "B.Cu") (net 3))
 (segment (start 131.005 102.7105) (end 139.04 94.6755) (width 0.2) (layer "F.Cu") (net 7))
 (segment (start 139.04 94.6755) (end 139.04 91.49) (width 0.2) (layer "F.Cu") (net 7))
 (segment (start 155.489 85.241) (end 155.59 85.14) (width 0.2) (layer "F.Cu") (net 31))
 (segment (start 157.52824 103.8615) (end 155.489 101.82226) (width 0.2) (layer "F.Cu") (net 31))
 (segment (start 155.489 101.82226) (end 155.489 85.241) (width 0.2) (layer "F.Cu") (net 31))
 (segment (start 160.545 102.7105) (end 159.394 103.8615) (width 0.2) (layer "F.Cu") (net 31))
 (segment (start 159.394 103.8615) (end 157.52824 103.8615) (width 0.2) (layer "F.Cu") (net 31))
 (segment (start 155.59 85.14) (end 156.54 85.14) (width 0.2) (layer "F.Cu") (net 31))
 (segment (start 157.49 77.52) (end 156.54 77.52) (width 0.2) (layer "F.Cu") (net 37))
 (segment (start 163.085 83.115) (end 157.49 77.52) (width 0.2) (layer "F.Cu") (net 37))
 (segment (start 163.085 102.7105) (end 163.085 83.115) (width 0.2) (layer "F.Cu") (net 37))
 (segment (start 152.24 97.26) (end 152.24 92.74) (width 0.2) (layer "F.Cu") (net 4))
 (segment (start 136.085 105.2505) (end 140.3345 109.5) (width 0.2) (layer "F.Cu") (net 4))
 (segment (start 145.5 104) (end 152.24 97.26) (width 0.2) (layer "F.Cu") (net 4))
 (segment (start 140.3345 109.5) (end 142.5 109.5) (width 0.2) (layer "F.Cu") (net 4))
 (via (at 145.5 104) (size 0.6) (drill 0.3) (layers "F.Cu" "B.Cu") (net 4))
 (via (at 142.5 109.5) (size 0.6) (drill 0.3) (layers "F.Cu" "B.Cu") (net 4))
 (segment (start 142.5 109.5) (end 145.5 106.5) (width 0.2) (layer "B.Cu") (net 4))
 (segment (start 145.5 106.5) (end 145.5 104) (width 0.2) (layer "B.Cu") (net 4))
 (segment (start 139.6375 104) (end 143.35 100.2875) (width 0.2) (layer "F.Cu") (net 6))
 (segment (start 133.545 105.2505) (end 134.7955 104) (width 0.2) (layer "F.Cu") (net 6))
 (segment (start 134.7955 104) (end 139.6375 104) (width 0.2) (layer "F.Cu") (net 6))
 (segment (start 143.35 100.2875) (end 143.35 92.74) (width 0.2) (layer "F.Cu") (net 6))
 (segment (start 159.5 101.5) (end 159.2155 101.5) (width 0.2) (layer "F.Cu") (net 32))
 (segment (start 156.54 83.87) (end 157.49 83.87) (width 0.2) (layer "F.Cu") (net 32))
 (segment (start 159.2155 101.5) (end 158.005 102.7105) (width 0.2) (layer "F.Cu") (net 32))
 (segment (start 162.684 98.316) (end 159.5 101.5) (width 0.2) (layer "F.Cu") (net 32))
 (segment (start 162.684 86.184) (end 162.684 98.316) (width 0.2) (layer "F.Cu") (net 32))
 (segment (start 158.62 85) (end 161.5 85) (width 0.2) (layer "F.Cu") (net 32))
 (segment (start 161.5 85) (end 162.684 86.184) (width 0.2) (layer "F.Cu") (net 32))
 (segment (start 157.49 83.87) (end 158.62 85) (width 0.2) (layer "F.Cu") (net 32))
 (segment (start 164.236 103.18726) (end 164.236 83.467) (width 0.2) (layer "F.Cu") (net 38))
 (segment (start 164.236 83.467) (end 157.019 76.25) (width 0.2) (layer "F.Cu") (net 38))
 (segment (start 163.32376 104.0995) (end 164.236 103.18726) (width 0.2) (layer "F.Cu") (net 38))
 (segment (start 161.696 104.0995) (end 163.32376 104.0995) (width 0.2) (layer "F.Cu") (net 38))
 (segment (start 157.019 76.25) (end 156.54 76.25) (width 0.2) (layer "F.Cu") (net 38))
 (segment (start 160.545 105.2505) (end 161.696 104.0995) (width 0.2) (layer "F.Cu") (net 38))
 (segment (start 169 92.5) (end 166 89.5) (width 0.2) (layer "F.Cu") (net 34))
 (segment (start 166.776 103.8615) (end 169 101.6375) (width 0.2) (layer "F.Cu") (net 34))
 (segment (start 163.085 105.2505) (end 164.474 103.8615) (width 0.2) (layer "F.Cu") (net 34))
 (segment (start 157.83 81.33) (end 156.54 81.33) (width 0.2) (layer "F.Cu") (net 34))
 (segment (start 169 101.6375) (end 169 92.5) (width 0.2) (layer "F.Cu") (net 34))
 (segment (start 164.474 103.8615) (end 166.776 103.8615) (width 0.2) (layer "F.Cu") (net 34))
 (segment (start 160.5 84) (end 157.83 81.33) (width 0.2) (layer "F.Cu") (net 34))
 (via (at 160.5 84) (size 0.6) (drill 0.3) (layers "F.Cu" "B.Cu") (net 34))
 (via (at 166 89.5) (size 0.6) (drill 0.3) (layers "F.Cu" "B.Cu") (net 34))
 (segment (start 166 89.5) (end 160.5 84) (width 0.2) (layer "B.Cu") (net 34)))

